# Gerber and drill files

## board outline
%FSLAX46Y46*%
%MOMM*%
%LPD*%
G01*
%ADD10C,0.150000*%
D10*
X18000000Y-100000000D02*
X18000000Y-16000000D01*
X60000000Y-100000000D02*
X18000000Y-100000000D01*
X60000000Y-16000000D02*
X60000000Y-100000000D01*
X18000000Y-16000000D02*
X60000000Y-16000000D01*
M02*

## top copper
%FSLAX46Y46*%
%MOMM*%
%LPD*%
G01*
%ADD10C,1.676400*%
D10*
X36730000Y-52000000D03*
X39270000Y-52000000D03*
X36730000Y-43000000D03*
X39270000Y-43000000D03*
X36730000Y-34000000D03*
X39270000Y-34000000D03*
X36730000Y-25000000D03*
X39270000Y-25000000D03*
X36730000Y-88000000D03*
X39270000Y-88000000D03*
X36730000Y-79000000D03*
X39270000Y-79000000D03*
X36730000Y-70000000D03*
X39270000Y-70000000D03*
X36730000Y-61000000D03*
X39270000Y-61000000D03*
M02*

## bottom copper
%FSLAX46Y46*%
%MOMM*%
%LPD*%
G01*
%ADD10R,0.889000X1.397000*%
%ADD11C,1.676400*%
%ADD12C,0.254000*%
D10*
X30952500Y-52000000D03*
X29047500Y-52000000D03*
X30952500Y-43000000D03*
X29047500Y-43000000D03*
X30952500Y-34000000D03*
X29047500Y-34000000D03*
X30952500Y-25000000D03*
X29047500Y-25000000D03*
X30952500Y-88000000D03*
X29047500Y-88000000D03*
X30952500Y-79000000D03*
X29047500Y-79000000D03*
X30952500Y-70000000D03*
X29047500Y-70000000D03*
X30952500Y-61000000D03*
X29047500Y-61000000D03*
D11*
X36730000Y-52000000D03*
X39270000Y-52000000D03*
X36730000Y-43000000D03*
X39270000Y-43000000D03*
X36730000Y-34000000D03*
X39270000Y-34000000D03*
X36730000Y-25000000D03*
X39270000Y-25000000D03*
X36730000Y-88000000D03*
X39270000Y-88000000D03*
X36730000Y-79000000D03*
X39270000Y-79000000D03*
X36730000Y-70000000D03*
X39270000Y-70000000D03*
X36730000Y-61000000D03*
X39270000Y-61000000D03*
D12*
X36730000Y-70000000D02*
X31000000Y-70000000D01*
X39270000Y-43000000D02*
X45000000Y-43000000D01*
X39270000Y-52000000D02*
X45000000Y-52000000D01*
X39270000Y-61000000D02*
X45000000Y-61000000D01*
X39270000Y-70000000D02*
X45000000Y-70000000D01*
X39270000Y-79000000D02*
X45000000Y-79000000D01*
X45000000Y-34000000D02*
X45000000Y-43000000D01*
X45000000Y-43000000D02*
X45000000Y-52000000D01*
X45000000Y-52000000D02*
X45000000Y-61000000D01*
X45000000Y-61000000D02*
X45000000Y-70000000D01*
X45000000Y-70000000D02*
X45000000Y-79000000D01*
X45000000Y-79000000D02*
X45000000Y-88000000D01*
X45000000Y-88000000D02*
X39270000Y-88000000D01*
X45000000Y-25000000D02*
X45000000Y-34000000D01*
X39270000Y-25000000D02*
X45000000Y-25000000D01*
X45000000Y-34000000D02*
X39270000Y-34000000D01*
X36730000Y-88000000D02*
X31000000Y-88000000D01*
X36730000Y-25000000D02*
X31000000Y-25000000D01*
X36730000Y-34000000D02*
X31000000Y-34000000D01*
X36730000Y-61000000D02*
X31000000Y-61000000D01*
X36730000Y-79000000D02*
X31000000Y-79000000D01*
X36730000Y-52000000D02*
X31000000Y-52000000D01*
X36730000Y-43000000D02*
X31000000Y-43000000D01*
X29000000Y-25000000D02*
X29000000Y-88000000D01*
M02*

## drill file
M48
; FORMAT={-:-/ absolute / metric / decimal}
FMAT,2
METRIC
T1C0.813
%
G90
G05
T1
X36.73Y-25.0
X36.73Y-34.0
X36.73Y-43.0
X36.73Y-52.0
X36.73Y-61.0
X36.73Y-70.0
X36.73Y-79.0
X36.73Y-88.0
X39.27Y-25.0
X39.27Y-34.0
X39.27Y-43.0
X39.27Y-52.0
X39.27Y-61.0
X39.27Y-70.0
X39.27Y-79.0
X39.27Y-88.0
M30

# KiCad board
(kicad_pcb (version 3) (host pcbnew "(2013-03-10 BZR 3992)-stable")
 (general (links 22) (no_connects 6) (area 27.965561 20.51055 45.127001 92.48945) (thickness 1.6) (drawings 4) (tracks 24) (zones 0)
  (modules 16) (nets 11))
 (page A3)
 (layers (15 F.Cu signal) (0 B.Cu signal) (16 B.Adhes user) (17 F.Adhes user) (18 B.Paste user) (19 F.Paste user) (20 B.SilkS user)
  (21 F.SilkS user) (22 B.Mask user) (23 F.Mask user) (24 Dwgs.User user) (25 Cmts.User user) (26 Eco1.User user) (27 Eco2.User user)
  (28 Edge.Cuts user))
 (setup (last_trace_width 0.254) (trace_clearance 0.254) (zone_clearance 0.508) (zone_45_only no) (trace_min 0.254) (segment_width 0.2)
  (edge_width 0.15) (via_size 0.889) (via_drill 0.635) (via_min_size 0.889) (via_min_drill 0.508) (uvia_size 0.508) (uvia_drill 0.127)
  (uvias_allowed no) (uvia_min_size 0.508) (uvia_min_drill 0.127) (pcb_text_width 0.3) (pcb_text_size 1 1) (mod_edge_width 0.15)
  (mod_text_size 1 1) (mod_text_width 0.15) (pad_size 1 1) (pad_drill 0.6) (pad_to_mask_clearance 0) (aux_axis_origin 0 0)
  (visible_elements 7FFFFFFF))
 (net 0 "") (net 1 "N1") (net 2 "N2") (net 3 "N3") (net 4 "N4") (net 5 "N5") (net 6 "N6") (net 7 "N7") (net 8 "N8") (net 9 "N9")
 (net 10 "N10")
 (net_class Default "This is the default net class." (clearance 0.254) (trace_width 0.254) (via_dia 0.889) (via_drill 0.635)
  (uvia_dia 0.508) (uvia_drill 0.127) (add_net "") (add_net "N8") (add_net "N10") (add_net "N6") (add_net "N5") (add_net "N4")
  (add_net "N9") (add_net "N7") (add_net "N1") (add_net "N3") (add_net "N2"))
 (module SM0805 (layer B.Cu) (at 30 52 180)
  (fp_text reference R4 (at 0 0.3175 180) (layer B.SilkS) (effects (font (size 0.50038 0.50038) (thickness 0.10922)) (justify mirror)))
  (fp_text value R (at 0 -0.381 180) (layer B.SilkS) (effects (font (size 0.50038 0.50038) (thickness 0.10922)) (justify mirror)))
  (pad 1 smd rect (at -0.9525 0 180) (size 0.889 1.397) (layers B.Cu B.Paste B.Mask) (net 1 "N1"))
  (pad 2 smd rect (at 0.9525 0 180) (size 0.889 1.397) (layers B.Cu B.Paste B.Mask) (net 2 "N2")))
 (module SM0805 (layer B.Cu) (at 30 43 180)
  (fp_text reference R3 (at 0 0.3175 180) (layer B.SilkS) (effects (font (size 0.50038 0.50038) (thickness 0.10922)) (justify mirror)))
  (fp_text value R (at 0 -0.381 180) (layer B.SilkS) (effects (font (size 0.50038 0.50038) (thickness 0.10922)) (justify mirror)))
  (pad 1 smd rect (at -0.9525 0 180) (size 0.889 1.397) (layers B.Cu B.Paste B.Mask) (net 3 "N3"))
  (pad 2 smd rect (at 0.9525 0 180) (size 0.889 1.397) (layers B.Cu B.Paste B.Mask) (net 2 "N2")))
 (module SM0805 (layer B.Cu) (at 30 34 180)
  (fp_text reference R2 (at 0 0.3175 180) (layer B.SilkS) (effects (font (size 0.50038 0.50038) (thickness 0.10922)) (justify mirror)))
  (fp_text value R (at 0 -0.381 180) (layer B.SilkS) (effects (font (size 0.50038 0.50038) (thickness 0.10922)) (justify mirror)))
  (pad 1 smd rect (at -0.9525 0 180) (size 0.889 1.397) (layers B.Cu B.Paste B.Mask) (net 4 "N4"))
  (pad 2 smd rect (at 0.9525 0 180) (size 0.889 1.397) (layers B.Cu B.Paste B.Mask) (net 2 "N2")))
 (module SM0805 (layer B.Cu) (at 30 25 180)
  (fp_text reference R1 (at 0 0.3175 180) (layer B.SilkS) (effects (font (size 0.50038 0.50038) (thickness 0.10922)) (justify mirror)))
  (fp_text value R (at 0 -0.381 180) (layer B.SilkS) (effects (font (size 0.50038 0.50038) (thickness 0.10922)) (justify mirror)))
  (pad 1 smd rect (at -0.9525 0 180) (size 0.889 1.397) (layers B.Cu B.Paste B.Mask) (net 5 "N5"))
  (pad 2 smd rect (at 0.9525 0 180) (size 0.889 1.397) (layers B.Cu B.Paste B.Mask) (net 2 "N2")))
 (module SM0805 (layer B.Cu) (at 30 88 180)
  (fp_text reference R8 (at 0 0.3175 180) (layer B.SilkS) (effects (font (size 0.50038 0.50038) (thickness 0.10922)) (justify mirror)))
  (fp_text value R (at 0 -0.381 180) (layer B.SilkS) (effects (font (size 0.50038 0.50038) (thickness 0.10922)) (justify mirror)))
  (pad 1 smd rect (at -0.9525 0 180) (size 0.889 1.397) (layers B.Cu B.Paste B.Mask) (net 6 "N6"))
  (pad 2 smd rect (at 0.9525 0 180) (size 0.889 1.397) (layers B.Cu B.Paste B.Mask) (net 2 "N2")))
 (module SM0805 (layer B.Cu) (at 30 79 180)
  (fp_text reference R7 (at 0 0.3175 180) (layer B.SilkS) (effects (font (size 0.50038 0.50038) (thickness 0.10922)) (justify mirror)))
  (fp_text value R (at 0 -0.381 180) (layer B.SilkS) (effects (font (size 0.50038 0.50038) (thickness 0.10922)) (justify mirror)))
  (pad 1 smd rect (at -0.9525 0 180) (size 0.889 1.397) (layers B.Cu B.Paste B.Mask) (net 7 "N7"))
  (pad 2 smd rect (at 0.9525 0 180) (size 0.889 1.397) (layers B.Cu B.Paste B.Mask) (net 2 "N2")))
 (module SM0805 (layer B.Cu) (at 30 70 180)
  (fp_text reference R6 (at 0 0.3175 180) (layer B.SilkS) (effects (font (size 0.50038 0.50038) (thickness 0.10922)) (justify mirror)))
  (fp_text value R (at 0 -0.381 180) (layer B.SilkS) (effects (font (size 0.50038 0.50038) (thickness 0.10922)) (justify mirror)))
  (pad 1 smd rect (at -0.9525 0 180) (size 0.889 1.397) (layers B.Cu B.Paste B.Mask) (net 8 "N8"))
  (pad 2 smd rect (at 0.9525 0 180) (size 0.889 1.397) (layers B.Cu B.Paste B.Mask) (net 2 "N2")))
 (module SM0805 (layer B.Cu) (at 30 61 180)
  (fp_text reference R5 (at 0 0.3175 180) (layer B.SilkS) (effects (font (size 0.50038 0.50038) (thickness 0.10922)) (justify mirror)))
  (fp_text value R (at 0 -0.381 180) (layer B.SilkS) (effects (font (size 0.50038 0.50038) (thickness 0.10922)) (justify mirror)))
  (pad 1 smd rect (at -0.9525 0 180) (size 0.889 1.397) (layers B.Cu B.Paste B.Mask) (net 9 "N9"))
  (pad 2 smd rect (at 0.9525 0 180) (size 0.889 1.397) (layers B.Cu B.Paste B.Mask) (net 2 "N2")))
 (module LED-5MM (layer F.Cu) (at 38 52)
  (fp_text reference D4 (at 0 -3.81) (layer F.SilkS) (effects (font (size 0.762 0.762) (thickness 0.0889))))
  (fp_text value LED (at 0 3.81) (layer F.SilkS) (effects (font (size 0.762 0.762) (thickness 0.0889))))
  (pad 1 thru_hole circle (at -1.27 0) (size 1.6764 1.6764) (drill 0.812799) (layers *.Cu *.Mask F.SilkS) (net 1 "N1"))
  (pad 2 thru_hole circle (at 1.27 0) (size 1.6764 1.6764) (drill 0.812799) (layers *.Cu *.Mask F.SilkS) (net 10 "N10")))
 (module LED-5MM (layer F.Cu) (at 38 43)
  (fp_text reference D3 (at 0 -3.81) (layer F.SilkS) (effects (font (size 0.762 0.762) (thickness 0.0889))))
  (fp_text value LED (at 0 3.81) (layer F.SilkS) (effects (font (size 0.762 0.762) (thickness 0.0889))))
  (pad 1 thru_hole circle (at -1.27 0) (size 1.6764 1.6764) (drill 0.812799) (layers *.Cu *.Mask F.SilkS) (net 3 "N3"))
  (pad 2 thru_hole circle (at 1.27 0) (size 1.6764 1.6764) (drill 0.812799) (layers *.Cu *.Mask F.SilkS) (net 10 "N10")))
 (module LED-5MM (layer F.Cu) (at 38 34)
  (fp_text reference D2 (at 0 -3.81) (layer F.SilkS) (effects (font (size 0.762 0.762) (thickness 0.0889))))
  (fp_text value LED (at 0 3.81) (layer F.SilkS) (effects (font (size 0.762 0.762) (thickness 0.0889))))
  (pad 1 thru_hole circle (at -1.27 0) (size 1.6764 1.6764) (drill 0.812799) (layers *.Cu *.Mask F.SilkS) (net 4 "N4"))
  (pad 2 thru_hole circle (at 1.27 0) (size 1.6764 1.6764) (drill 0.812799) (layers *.Cu *.Mask F.SilkS) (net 10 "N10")))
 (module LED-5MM (layer F.Cu) (at 38 25)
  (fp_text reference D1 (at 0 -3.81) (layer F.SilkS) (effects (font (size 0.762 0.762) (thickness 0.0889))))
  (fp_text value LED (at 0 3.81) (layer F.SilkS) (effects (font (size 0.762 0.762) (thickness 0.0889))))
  (pad 1 thru_hole circle (at -1.27 0) (size 1.6764 1.6764) (drill 0.812799) (layers *.Cu *.Mask F.SilkS) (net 5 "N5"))
  (pad 2 thru_hole circle (at 1.27 0) (size 1.6764 1.6764) (drill 0.812799) (layers *.Cu *.Mask F.SilkS) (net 10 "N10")))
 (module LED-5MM (layer F.Cu) (at 38 88)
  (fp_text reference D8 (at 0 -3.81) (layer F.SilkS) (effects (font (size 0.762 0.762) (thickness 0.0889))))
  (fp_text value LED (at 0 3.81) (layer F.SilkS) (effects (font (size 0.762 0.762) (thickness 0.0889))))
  (pad 1 thru_hole circle (at -1.27 0) (size 1.6764 1.6764) (drill 0.812799) (layers *.Cu *.Mask F.SilkS) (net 6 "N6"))
  (pad 2 thru_hole circle (at 1.27 0) (size 1.6764 1.6764) (drill 0.812799) (layers *.Cu *.Mask F.SilkS) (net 10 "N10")))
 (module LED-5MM (layer F.Cu) (at 38 79)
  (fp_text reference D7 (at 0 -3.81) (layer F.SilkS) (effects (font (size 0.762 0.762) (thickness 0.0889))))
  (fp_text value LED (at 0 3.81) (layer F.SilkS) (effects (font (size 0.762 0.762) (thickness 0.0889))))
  (pad 1 thru_hole circle (at -1.27 0) (size 1.6764 1.6764) (drill 0.812799) (layers *.Cu *.Mask F.SilkS) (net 7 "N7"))
  (pad 2 thru_hole circle (at 1.27 0) (size 1.6764 1.6764) (drill 0.812799) (layers *.Cu *.Mask F.SilkS) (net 10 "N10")))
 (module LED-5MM (layer F.Cu) (at 38 70)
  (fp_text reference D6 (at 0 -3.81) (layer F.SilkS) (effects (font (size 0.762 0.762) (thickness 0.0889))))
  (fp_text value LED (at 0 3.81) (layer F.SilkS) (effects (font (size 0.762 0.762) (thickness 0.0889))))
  (pad 1 thru_hole circle (at -1.27 0) (size 1.6764 1.6764) (drill 0.812799) (layers *.Cu *.Mask F.SilkS) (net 8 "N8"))
  (pad 2 thru_hole circle (at 1.27 0) (size 1.6764 1.6764) (drill 0.812799) (layers *.Cu *.Mask F.SilkS) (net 10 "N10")))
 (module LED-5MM (layer F.Cu) (at 38 61)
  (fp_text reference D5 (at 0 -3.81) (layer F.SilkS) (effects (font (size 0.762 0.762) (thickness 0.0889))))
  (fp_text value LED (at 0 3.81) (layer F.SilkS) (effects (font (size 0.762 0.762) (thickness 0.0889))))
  (pad 1 thru_hole circle (at -1.27 0) (size 1.6764 1.6764) (drill 0.812799) (layers *.Cu *.Mask F.SilkS) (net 9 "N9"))
  (pad 2 thru_hole circle (at 1.27 0) (size 1.6764 1.6764) (drill 0.812799) (layers *.Cu *.Mask F.SilkS) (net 10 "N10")))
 (gr_line (start 18 100) (end 18 16) (angle 90) (layer Edge.Cuts) (width 0.15))
 (gr_line (start 60 100) (end 18 100) (angle 90) (layer Edge.Cuts) (width 0.15))
 (gr_line (start 60 16) (end 60 100) (angle 90) (layer Edge.Cuts) (width 0.15))
 (gr_line (start 18 16) (end 60 16) (angle 90) (layer Edge.Cuts) (width 0.15))
 (segment (start 36.73 70) (end 31 70) (width 0.254) (layer B.Cu) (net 8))
 (segment (start 39.27 43) (end 45 43) (width 0.254) (layer B.Cu) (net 10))
 (segment (start 39.27 52) (end 45 52) (width 0.254) (layer B.Cu) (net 10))
 (segment (start 39.27 61) (end 45 61) (width 0.254) (layer B.Cu) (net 10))
 (segment (start 39.27 70) (end 45 70) (width 0.254) (layer B.Cu) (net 10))
 (segment (start 39.27 79) (end 45 79) (width 0.254) (layer B.Cu) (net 10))
 (segment (start 45 34) (end 45 43) (width 0.254) (layer B.Cu) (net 10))
 (segment (start 45 43) (end 45 52) (width 0.254) (layer B.Cu) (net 10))
 (segment (start 45 52) (end 45 61) (width 0.254) (layer B.Cu) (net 10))
 (segment (start 45 61) (end 45 70) (width 0.254) (layer B.Cu) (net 10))
 (segment (start 45 70) (end 45 79) (width 0.254) (layer B.Cu) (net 10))
 (segment (start 45 79) (end 45 88) (width 0.254) (layer B.Cu) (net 10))
 (segment (start 45 88) (end 39.27 88) (width 0.254) (layer B.Cu) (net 10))
 (segment (start 45 25) (end 45 34) (width 0.254) (layer B.Cu) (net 10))
 (segment (start 39.27 25) (end 45 25) (width 0.254) (layer B.Cu) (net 10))
 (segment (start 45 34) (end 39.27 34) (width 0.254) (layer B.Cu) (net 10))
 (segment (start 36.73 88) (end 31 88) (width 0.254) (layer B.Cu) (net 6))
 (segment (start 36.73 25) (end 31 25) (width 0.254) (layer B.Cu) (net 5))
 (segment (start 36.73 34) (end 31 34) (width 0.254) (layer B.Cu) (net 4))
 (segment (start 36.73 61) (end 31 61) (width 0.254) (layer B.Cu) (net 9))
 (segment (start 36.73 79) (end 31 79) (width 0.254) (layer B.Cu) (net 7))
 (segment (start 36.73 52) (end 31 52) (width 0.254) (layer B.Cu) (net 1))
 (segment (start 36.73 43) (end 31 43) (width 0.254) (layer B.Cu) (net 3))
 (segment (start 29 25) (end 29 88) (width 0.254) (layer B.Cu) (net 2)))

